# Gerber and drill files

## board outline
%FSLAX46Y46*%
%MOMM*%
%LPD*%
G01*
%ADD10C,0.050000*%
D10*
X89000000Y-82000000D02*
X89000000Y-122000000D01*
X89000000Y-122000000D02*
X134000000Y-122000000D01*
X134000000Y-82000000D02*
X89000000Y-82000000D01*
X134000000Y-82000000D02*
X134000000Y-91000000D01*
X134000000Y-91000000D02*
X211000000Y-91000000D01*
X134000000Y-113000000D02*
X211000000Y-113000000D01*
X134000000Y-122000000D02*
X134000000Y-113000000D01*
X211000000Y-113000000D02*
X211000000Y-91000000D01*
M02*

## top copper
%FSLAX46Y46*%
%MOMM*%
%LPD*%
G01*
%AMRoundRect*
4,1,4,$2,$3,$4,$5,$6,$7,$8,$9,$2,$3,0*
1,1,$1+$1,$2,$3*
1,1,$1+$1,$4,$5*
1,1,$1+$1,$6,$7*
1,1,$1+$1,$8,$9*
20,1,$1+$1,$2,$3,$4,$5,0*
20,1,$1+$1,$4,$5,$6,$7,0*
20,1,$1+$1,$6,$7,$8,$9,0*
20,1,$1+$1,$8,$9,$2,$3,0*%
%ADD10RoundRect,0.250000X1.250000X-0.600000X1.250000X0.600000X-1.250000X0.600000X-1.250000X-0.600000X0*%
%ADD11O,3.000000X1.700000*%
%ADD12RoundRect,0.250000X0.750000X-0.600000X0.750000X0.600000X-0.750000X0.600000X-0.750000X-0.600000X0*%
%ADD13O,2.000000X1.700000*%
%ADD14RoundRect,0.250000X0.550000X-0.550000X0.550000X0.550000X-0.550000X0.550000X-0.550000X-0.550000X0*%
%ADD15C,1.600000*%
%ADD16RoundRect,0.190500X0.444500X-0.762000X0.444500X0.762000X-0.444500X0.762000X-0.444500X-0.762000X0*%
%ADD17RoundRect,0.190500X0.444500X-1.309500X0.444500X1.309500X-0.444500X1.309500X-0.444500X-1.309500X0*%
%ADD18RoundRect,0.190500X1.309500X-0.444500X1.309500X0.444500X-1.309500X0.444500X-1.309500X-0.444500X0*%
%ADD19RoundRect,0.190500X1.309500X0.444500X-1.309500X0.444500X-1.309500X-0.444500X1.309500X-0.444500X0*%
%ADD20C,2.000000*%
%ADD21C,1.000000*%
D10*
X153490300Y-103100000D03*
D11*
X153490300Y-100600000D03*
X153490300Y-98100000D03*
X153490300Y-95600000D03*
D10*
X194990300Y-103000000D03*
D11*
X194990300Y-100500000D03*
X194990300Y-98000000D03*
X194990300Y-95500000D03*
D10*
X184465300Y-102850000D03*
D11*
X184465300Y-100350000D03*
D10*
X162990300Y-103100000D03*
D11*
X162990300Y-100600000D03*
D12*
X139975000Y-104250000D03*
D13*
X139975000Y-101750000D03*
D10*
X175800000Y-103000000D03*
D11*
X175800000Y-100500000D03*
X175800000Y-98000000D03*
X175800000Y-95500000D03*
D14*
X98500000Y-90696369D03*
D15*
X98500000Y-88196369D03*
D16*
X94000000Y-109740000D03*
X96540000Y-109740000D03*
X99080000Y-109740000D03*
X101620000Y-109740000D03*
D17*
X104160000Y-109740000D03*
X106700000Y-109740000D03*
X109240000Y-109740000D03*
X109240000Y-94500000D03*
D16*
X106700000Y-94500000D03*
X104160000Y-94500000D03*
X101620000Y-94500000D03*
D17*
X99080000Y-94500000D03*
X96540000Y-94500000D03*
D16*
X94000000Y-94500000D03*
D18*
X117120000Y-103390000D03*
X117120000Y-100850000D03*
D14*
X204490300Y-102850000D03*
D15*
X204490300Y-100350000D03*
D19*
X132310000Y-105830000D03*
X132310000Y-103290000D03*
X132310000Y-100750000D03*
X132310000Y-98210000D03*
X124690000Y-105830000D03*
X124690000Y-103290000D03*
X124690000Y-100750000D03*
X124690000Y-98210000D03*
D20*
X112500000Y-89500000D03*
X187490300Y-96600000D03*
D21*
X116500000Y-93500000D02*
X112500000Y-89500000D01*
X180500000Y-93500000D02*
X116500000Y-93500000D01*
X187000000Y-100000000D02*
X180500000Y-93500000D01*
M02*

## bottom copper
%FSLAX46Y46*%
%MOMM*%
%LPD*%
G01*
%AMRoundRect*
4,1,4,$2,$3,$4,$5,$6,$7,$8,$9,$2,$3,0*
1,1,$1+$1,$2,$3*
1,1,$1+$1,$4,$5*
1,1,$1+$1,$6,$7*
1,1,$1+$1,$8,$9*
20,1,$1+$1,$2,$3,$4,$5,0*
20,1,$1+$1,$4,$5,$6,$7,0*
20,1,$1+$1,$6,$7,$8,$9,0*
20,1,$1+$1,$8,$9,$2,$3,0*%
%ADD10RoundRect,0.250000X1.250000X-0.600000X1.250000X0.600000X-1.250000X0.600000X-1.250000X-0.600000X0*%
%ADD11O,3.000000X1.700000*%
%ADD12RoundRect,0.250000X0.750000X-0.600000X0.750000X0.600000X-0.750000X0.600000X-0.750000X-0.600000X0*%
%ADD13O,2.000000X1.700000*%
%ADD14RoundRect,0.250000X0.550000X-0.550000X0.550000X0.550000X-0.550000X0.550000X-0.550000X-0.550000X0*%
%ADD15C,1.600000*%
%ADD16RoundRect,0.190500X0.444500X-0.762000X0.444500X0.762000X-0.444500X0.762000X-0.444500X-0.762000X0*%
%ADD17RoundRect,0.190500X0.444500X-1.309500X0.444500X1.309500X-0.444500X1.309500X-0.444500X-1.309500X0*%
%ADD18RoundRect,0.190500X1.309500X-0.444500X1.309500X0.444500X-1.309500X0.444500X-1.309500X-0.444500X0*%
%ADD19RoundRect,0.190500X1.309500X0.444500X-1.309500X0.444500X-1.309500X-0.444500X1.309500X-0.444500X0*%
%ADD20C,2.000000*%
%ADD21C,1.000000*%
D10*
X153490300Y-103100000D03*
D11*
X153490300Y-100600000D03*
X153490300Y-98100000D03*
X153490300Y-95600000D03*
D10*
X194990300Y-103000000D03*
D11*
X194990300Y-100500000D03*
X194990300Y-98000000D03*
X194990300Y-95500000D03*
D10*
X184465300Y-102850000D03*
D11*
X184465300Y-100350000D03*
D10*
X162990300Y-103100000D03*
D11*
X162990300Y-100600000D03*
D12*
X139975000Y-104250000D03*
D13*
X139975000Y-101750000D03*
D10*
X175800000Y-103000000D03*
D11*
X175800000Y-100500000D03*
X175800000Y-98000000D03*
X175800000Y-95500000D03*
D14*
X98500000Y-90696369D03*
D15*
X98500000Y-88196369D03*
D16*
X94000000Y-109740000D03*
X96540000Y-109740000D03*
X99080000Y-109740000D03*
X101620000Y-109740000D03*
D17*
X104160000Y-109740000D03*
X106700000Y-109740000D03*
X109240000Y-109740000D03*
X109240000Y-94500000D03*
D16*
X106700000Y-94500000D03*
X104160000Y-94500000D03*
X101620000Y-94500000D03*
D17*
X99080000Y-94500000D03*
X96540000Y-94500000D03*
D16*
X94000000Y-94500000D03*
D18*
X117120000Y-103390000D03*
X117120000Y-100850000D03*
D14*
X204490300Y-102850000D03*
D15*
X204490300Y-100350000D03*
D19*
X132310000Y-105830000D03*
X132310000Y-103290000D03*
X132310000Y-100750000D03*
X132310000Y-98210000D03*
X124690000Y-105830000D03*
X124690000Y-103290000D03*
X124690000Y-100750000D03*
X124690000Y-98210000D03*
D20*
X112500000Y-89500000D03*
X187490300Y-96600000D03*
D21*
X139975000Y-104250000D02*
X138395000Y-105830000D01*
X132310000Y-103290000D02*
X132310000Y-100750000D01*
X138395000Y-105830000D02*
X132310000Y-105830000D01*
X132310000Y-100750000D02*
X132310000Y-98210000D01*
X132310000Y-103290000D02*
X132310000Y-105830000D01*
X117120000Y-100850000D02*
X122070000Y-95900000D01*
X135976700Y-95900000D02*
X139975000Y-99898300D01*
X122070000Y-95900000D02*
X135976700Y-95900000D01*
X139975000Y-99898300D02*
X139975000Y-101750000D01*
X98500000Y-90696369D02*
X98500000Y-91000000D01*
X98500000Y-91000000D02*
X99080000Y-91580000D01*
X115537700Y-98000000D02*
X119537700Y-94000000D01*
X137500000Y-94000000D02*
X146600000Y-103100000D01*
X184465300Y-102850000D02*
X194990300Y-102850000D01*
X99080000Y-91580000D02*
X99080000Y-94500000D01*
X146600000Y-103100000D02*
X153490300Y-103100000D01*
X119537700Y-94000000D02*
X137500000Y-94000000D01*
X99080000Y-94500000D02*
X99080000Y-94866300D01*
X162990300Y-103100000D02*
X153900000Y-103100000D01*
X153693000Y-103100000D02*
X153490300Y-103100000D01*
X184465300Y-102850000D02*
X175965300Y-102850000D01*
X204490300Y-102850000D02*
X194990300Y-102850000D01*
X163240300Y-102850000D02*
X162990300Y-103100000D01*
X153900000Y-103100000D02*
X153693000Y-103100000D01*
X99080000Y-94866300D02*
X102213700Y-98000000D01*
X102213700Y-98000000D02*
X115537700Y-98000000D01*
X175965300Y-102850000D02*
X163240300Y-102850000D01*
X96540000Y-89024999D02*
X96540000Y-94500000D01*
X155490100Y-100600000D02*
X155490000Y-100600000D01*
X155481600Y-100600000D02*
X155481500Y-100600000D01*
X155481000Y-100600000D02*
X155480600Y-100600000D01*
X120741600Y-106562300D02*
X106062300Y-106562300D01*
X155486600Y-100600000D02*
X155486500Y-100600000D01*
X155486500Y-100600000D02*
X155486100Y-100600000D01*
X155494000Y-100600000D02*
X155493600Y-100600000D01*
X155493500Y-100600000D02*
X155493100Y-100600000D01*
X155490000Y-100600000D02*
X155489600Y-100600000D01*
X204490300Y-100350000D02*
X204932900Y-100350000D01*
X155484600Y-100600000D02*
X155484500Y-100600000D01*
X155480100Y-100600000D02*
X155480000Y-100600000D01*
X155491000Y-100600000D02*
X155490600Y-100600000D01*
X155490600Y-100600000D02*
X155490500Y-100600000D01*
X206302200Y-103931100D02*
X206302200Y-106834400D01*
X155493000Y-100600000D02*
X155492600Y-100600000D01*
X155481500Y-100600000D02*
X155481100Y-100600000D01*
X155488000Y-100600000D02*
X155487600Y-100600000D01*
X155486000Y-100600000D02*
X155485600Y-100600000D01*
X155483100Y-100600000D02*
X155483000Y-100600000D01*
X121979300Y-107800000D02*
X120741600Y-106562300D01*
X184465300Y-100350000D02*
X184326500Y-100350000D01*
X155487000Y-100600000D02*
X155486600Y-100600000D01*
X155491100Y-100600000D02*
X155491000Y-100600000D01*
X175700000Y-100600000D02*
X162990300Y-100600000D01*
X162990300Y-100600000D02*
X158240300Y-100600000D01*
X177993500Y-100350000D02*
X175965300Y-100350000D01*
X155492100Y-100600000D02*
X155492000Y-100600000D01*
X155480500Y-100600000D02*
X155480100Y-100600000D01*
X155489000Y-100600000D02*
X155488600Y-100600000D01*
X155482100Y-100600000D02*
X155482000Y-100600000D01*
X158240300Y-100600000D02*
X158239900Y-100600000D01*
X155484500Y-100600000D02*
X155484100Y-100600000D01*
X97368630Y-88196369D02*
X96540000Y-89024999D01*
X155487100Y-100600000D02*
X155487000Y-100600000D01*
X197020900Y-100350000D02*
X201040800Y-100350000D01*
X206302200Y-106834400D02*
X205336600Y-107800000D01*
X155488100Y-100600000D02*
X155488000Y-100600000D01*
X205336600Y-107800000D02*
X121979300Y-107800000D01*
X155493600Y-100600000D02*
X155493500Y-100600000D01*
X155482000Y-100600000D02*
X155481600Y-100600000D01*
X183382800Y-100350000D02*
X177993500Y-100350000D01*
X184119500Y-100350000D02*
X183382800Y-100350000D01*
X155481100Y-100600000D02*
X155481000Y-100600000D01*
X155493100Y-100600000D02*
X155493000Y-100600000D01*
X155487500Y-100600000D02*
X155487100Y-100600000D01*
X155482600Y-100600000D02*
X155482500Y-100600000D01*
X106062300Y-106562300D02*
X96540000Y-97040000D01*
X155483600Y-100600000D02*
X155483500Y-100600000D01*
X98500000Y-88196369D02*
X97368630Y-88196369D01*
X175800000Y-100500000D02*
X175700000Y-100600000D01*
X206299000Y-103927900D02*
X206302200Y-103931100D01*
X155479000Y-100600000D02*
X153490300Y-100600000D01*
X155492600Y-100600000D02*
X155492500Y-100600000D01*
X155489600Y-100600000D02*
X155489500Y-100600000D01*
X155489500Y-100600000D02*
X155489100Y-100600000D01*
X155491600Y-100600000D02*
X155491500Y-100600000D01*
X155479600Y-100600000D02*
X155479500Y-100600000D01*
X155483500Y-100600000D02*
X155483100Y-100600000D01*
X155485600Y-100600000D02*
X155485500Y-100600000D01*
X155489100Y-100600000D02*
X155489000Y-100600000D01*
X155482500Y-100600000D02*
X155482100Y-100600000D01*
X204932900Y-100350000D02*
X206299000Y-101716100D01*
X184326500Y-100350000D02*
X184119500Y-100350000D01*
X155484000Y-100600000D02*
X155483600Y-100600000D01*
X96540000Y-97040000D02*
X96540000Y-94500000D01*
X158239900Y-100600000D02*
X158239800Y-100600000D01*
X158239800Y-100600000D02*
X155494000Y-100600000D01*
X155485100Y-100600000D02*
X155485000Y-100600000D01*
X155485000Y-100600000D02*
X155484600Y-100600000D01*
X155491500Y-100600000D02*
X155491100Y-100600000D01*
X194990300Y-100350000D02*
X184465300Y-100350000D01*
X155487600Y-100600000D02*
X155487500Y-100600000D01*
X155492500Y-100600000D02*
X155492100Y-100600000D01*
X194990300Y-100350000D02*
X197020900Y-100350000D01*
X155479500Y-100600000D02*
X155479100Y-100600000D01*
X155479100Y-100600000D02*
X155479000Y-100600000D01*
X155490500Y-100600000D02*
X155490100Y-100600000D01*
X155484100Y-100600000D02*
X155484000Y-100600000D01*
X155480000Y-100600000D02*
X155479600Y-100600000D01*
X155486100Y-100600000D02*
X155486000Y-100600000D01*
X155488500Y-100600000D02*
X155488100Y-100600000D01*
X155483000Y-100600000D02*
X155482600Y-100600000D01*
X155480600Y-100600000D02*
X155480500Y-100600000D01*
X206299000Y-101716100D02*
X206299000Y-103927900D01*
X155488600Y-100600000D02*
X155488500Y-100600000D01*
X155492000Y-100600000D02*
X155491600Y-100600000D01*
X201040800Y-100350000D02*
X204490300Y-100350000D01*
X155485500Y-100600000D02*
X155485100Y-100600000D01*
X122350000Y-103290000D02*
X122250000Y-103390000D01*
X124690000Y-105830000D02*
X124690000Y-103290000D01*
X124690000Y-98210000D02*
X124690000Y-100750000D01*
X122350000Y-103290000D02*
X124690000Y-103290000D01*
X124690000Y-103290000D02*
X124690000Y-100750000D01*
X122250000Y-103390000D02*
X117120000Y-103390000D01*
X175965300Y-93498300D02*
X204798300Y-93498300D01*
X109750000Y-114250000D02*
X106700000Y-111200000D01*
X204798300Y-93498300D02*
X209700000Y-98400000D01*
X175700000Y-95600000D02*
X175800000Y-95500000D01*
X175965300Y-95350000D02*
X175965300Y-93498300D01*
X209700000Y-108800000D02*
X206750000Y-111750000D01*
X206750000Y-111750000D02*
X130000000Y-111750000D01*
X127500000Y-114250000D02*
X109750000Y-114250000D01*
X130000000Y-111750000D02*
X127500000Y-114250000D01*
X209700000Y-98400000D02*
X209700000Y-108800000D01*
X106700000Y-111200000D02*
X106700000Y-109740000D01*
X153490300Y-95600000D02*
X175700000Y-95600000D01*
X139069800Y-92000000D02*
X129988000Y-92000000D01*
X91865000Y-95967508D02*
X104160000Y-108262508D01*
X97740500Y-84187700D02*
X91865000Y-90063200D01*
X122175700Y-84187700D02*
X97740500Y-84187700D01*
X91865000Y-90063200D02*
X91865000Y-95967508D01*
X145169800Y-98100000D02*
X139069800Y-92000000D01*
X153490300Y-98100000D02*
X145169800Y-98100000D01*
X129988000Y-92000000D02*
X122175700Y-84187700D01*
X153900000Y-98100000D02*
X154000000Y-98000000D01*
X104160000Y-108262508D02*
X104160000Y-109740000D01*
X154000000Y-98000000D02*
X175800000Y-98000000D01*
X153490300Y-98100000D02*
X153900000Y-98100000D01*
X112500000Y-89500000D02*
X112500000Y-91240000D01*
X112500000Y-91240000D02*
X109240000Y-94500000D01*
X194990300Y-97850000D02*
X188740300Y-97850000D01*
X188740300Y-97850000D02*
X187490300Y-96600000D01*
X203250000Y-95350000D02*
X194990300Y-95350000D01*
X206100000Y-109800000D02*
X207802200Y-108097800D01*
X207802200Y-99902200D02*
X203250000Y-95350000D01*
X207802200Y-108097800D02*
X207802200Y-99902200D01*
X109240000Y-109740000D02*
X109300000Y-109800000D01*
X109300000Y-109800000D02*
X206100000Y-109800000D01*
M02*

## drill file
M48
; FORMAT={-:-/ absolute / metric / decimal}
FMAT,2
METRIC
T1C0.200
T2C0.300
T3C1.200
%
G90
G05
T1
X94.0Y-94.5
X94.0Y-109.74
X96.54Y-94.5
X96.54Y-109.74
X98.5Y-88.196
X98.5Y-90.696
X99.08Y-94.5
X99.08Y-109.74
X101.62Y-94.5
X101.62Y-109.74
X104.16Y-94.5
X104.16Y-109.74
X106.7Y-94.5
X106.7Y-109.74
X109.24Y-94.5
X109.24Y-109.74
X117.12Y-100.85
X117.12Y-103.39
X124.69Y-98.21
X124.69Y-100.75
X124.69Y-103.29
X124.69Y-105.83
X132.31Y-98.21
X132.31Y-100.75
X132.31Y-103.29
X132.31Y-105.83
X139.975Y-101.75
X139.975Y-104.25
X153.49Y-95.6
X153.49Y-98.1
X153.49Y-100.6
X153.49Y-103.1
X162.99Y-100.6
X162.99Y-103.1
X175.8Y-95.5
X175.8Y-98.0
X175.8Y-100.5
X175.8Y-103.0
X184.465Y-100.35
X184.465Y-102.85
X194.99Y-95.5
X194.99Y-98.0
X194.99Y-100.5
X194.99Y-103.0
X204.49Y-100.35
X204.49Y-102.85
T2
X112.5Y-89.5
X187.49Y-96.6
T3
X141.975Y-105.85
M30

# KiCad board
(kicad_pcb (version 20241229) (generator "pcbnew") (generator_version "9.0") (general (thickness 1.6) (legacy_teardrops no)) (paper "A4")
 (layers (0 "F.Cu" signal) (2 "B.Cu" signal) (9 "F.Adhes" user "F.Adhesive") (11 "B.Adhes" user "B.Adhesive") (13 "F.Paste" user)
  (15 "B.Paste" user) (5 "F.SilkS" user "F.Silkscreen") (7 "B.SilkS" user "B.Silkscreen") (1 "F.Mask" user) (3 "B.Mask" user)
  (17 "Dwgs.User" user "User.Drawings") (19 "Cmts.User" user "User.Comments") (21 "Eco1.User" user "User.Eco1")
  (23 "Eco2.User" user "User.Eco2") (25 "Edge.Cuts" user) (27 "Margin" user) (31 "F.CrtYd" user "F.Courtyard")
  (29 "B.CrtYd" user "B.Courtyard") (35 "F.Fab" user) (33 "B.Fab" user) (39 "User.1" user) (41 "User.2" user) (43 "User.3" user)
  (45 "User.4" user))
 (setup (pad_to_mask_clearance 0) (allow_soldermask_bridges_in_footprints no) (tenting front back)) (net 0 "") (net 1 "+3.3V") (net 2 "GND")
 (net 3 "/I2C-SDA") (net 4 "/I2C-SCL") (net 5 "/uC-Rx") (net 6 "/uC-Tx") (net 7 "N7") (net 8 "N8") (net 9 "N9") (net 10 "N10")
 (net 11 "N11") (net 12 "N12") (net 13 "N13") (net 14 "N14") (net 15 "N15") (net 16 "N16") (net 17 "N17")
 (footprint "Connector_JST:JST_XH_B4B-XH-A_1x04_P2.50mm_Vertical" (layer "F.Cu") (at 153.4903 103.1 90)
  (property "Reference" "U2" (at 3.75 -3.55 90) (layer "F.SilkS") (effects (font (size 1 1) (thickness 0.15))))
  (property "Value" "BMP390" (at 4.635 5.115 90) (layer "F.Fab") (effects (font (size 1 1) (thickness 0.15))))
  (pad "1" thru_hole roundrect (at 0 0 90) (size 1.7 3) (drill 0.2) (layers "*.Cu" "*.Mask") (remove_unused_layers no)
   (roundrect_rratio 0.147059) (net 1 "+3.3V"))
  (pad "2" thru_hole oval (at 2.5 0 90) (size 1.7 3) (drill 0.2) (layers "*.Cu" "*.Mask") (remove_unused_layers no) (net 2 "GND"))
  (pad "3" thru_hole oval (at 5 0 90) (size 1.7 3) (drill 0.2) (layers "*.Cu" "*.Mask") (remove_unused_layers no) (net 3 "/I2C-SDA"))
  (pad "4" thru_hole oval (at 7.5 0 90) (size 1.7 3) (drill 0.2) (layers "*.Cu" "*.Mask") (remove_unused_layers no) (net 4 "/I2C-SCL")))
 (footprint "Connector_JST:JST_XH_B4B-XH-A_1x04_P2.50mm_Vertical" (layer "F.Cu") (at 194.9903 103 90)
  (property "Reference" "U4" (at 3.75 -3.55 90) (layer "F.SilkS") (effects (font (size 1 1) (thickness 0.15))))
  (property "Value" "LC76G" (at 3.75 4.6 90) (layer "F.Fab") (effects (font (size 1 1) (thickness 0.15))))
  (pad "1" thru_hole roundrect (at 0 0 90) (size 1.7 3) (drill 0.2) (layers "*.Cu" "*.Mask") (remove_unused_layers no)
   (roundrect_rratio 0.147059) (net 1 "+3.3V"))
  (pad "2" thru_hole oval (at 2.5 0 90) (size 1.7 3) (drill 0.2) (layers "*.Cu" "*.Mask") (remove_unused_layers no) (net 2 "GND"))
  (pad "3" thru_hole oval (at 5 0 90) (size 1.7 3) (drill 0.2) (layers "*.Cu" "*.Mask") (remove_unused_layers no) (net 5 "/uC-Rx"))
  (pad "4" thru_hole oval (at 7.5 0 90) (size 1.7 3) (drill 0.2) (layers "*.Cu" "*.Mask") (remove_unused_layers no) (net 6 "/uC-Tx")))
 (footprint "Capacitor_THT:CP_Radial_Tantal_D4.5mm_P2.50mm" (layer "F.Cu") (at 184.4653 102.85 90)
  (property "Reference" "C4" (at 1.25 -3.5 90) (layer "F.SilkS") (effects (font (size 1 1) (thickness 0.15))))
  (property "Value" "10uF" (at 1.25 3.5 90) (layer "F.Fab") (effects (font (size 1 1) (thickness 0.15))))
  (pad "1" thru_hole roundrect (at 0 0 90) (size 1.7 3) (drill 0.2) (layers "*.Cu" "*.Mask") (remove_unused_layers no)
   (roundrect_rratio 0.147059) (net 1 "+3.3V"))
  (pad "2" thru_hole oval (at 2.5 0 90) (size 1.7 3) (drill 0.2) (layers "*.Cu" "*.Mask") (remove_unused_layers no) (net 2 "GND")))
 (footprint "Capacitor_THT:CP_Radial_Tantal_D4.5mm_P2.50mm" (layer "F.Cu") (at 162.9903 103.1 90)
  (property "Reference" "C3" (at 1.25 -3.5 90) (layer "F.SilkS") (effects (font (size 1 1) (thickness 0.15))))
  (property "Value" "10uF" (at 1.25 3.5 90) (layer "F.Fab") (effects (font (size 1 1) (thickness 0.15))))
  (pad "1" thru_hole roundrect (at 0 0 90) (size 1.7 3) (drill 0.2) (layers "*.Cu" "*.Mask") (remove_unused_layers no)
   (roundrect_rratio 0.147059) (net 1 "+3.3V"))
  (pad "2" thru_hole oval (at 2.5 0 90) (size 1.7 3) (drill 0.2) (layers "*.Cu" "*.Mask") (remove_unused_layers no) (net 2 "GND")))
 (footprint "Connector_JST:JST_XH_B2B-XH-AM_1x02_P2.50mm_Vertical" (layer "F.Cu") (at 139.975 104.25 90)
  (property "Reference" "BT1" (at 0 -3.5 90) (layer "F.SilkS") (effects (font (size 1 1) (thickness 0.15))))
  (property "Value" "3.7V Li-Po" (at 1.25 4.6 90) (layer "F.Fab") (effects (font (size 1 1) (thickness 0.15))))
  (pad "" np_thru_hole circle (at -1.6 2 90) (size 1.2 1.2) (drill 1.2) (layers "*.Cu" "*.Mask"))
  (pad "1" thru_hole roundrect (at 0 0 90) (size 1.7 2) (drill 0.2) (layers "*.Cu" "*.Mask") (remove_unused_layers no)
   (roundrect_rratio 0.147059) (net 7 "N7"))
  (pad "2" thru_hole oval (at 2.5 0 90) (size 1.7 2) (drill 0.2) (layers "*.Cu" "*.Mask") (remove_unused_layers no) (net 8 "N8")))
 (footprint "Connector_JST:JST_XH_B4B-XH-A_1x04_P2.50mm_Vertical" (layer "F.Cu") (at 175.8 103 90)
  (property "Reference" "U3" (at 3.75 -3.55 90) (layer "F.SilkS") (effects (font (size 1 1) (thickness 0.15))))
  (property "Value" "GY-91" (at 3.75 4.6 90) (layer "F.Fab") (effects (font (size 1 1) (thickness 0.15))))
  (pad "1" thru_hole roundrect (at 0 0 90) (size 1.7 3) (drill 0.2) (layers "*.Cu" "*.Mask") (remove_unused_layers no)
   (roundrect_rratio 0.147059) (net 1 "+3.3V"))
  (pad "2" thru_hole oval (at 2.5 0 90) (size 1.7 3) (drill 0.2) (layers "*.Cu" "*.Mask") (remove_unused_layers no) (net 2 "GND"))
  (pad "3" thru_hole oval (at 5 0 90) (size 1.7 3) (drill 0.2) (layers "*.Cu" "*.Mask") (remove_unused_layers no) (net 3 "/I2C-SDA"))
  (pad "4" thru_hole oval (at 7.5 0 90) (size 1.7 3) (drill 0.2) (layers "*.Cu" "*.Mask") (remove_unused_layers no) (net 4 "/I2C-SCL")))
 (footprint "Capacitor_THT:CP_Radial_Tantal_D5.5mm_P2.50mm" (layer "F.Cu") (at 98.5 90.696369 90)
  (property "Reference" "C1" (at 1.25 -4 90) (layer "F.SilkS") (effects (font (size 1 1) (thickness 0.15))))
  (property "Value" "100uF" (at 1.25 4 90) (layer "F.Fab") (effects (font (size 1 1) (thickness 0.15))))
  (pad "1" thru_hole roundrect (at 0 0 90) (size 1.6 1.6) (drill 0.2) (layers "*.Cu" "*.Mask") (remove_unused_layers no)
   (roundrect_rratio 0.15625) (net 1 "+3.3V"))
  (pad "2" thru_hole circle (at 2.5 0 90) (size 1.6 1.6) (drill 0.2) (layers "*.Cu" "*.Mask") (remove_unused_layers no) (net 2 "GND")))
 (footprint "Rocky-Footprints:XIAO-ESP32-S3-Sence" (layer "F.Cu") (at 101.62 102.12 90)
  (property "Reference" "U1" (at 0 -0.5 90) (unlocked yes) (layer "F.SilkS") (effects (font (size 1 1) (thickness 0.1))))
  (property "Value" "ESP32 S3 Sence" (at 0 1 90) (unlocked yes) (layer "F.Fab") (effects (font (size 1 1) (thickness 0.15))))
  (pad "1" thru_hole roundrect (at -7.62 -7.62 90) (size 1.905 1.27) (drill 0.2) (layers "*.Cu" "*.Mask") (remove_unused_layers no)
   (roundrect_rratio 0.15) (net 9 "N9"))
  (pad "2" thru_hole roundrect (at -7.62 -5.08 90) (size 1.905 1.27) (drill 0.2) (layers "*.Cu" "*.Mask") (remove_unused_layers no)
   (roundrect_rratio 0.15) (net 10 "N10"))
  (pad "3" thru_hole roundrect (at -7.62 -2.54 90) (size 1.905 1.27) (drill 0.2) (layers "*.Cu" "*.Mask") (remove_unused_layers no)
   (roundrect_rratio 0.15) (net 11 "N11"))
  (pad "4" thru_hole roundrect (at -7.62 0 90) (size 1.905 1.27) (drill 0.2) (layers "*.Cu" "*.Mask") (remove_unused_layers no)
   (roundrect_rratio 0.15) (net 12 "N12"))
  (pad "5" thru_hole roundrect (at -7.62 2.54 90) (size 3 1.27) (drill 0.2) (layers "*.Cu" "*.Mask") (remove_unused_layers no)
   (roundrect_rratio 0.15) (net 3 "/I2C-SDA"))
  (pad "6" thru_hole roundrect (at -7.62 5.08 90) (size 3 1.27) (drill 0.2) (layers "*.Cu" "*.Mask") (remove_unused_layers no)
   (roundrect_rratio 0.15) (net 4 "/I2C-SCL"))
  (pad "7" thru_hole roundrect (at -7.62 7.62 90) (size 3 1.27) (drill 0.2) (layers "*.Cu" "*.Mask") (remove_unused_layers no)
   (roundrect_rratio 0.15) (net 6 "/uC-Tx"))
  (pad "8" thru_hole roundrect (at 7.62 7.62 90) (size 3 1.27) (drill 0.2) (layers "*.Cu" "*.Mask") (remove_unused_layers no)
   (roundrect_rratio 0.15) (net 5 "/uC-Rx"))
  (pad "9" thru_hole roundrect (at 7.62 5.08 90) (size 1.905 1.27) (drill 0.2) (layers "*.Cu" "*.Mask") (remove_unused_layers no)
   (roundrect_rratio 0.15) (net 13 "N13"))
  (pad "10" thru_hole roundrect (at 7.62 2.54 90) (size 1.905 1.27) (drill 0.2) (layers "*.Cu" "*.Mask") (remove_unused_layers no)
   (roundrect_rratio 0.15) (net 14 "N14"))
  (pad "11" thru_hole roundrect (at 7.62 0 90) (size 1.905 1.27) (drill 0.2) (layers "*.Cu" "*.Mask") (remove_unused_layers no)
   (roundrect_rratio 0.15) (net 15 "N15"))
  (pad "12" thru_hole roundrect (at 7.62 -2.54 90) (size 3 1.27) (drill 0.2) (layers "*.Cu" "*.Mask") (remove_unused_layers no)
   (roundrect_rratio 0.15) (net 1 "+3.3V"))
  (pad "13" thru_hole roundrect (at 7.62 -5.08 90) (size 3 1.27) (drill 0.2) (layers "*.Cu" "*.Mask") (remove_unused_layers no)
   (roundrect_rratio 0.15) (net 2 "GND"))
  (pad "14" thru_hole roundrect (at 7.62 -7.62 90) (size 1.905 1.27) (drill 0.2) (layers "*.Cu" "*.Mask") (remove_unused_layers no)
   (roundrect_rratio 0.15) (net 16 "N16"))
  (pad "15" thru_hole roundrect (at -1.27 15.5 90) (size 1.27 3) (drill 0.2) (layers "*.Cu" "*.Mask") (remove_unused_layers no)
   (roundrect_rratio 0.15) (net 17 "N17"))
  (pad "16" thru_hole roundrect (at 1.27 15.5 90) (size 1.27 3) (drill 0.2) (layers "*.Cu" "*.Mask") (remove_unused_layers no)
   (roundrect_rratio 0.15) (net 8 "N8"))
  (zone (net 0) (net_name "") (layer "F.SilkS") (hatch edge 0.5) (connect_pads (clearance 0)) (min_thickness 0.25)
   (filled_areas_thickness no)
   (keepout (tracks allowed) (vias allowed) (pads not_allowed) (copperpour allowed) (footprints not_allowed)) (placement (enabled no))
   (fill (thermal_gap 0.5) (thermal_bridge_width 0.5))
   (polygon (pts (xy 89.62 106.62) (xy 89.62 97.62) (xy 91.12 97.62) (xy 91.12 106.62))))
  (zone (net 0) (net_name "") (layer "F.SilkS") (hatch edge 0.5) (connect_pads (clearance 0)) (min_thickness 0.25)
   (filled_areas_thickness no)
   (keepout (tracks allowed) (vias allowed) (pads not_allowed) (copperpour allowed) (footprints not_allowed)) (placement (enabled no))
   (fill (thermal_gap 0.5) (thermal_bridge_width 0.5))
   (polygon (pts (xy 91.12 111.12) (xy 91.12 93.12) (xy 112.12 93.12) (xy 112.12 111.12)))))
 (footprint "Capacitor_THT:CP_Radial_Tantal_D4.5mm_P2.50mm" (layer "F.Cu") (at 204.4903 102.85 90)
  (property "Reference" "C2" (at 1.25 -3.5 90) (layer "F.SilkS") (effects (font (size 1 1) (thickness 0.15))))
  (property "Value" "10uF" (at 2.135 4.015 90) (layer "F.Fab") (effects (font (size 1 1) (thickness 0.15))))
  (pad "1" thru_hole roundrect (at 0 0 90) (size 1.6 1.6) (drill 0.2) (layers "*.Cu" "*.Mask") (remove_unused_layers no)
   (roundrect_rratio 0.15625) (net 1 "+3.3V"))
  (pad "2" thru_hole circle (at 2.5 0 90) (size 1.6 1.6) (drill 0.2) (layers "*.Cu" "*.Mask") (remove_unused_layers no) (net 2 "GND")))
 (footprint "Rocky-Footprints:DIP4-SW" (layer "F.Cu") (at 128.5 100.75 180)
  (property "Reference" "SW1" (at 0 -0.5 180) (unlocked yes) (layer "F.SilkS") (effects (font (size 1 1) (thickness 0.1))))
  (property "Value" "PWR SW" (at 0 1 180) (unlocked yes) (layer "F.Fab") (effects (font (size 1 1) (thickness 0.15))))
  (pad "1" thru_hole roundrect (at -3.81 -5.08 180) (size 3 1.27) (drill 0.2) (layers "*.Cu" "*.Mask") (remove_unused_layers no)
   (roundrect_rratio 0.15) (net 7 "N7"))
  (pad "1" thru_hole roundrect (at -3.81 -2.54 180) (size 3 1.27) (drill 0.2) (layers "*.Cu" "*.Mask") (remove_unused_layers no)
   (roundrect_rratio 0.15) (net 7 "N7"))
  (pad "1" thru_hole roundrect (at -3.81 0 180) (size 3 1.27) (drill 0.2) (layers "*.Cu" "*.Mask") (remove_unused_layers no)
   (roundrect_rratio 0.15) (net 7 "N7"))
  (pad "1" thru_hole roundrect (at -3.81 2.54 180) (size 3 1.27) (drill 0.2) (layers "*.Cu" "*.Mask") (remove_unused_layers no)
   (roundrect_rratio 0.15) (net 7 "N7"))
  (pad "2" thru_hole roundrect (at 3.81 -5.08 180) (size 3 1.27) (drill 0.2) (layers "*.Cu" "*.Mask") (remove_unused_layers no)
   (roundrect_rratio 0.15) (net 17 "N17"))
  (pad "2" thru_hole roundrect (at 3.81 -2.54 180) (size 3 1.27) (drill 0.2) (layers "*.Cu" "*.Mask") (remove_unused_layers no)
   (roundrect_rratio 0.15) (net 17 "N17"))
  (pad "2" thru_hole roundrect (at 3.81 0 180) (size 3 1.27) (drill 0.2) (layers "*.Cu" "*.Mask") (remove_unused_layers no)
   (roundrect_rratio 0.15) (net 17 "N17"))
  (pad "2" thru_hole roundrect (at 3.81 2.54 180) (size 3 1.27) (drill 0.2) (layers "*.Cu" "*.Mask") (remove_unused_layers no)
   (roundrect_rratio 0.15) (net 17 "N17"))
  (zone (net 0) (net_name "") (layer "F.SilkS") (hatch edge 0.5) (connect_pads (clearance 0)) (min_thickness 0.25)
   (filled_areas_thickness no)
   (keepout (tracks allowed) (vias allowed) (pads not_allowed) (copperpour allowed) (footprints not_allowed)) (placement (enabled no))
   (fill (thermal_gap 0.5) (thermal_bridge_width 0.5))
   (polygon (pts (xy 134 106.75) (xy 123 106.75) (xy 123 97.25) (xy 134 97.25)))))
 (gr_line (start 89 82) (end 89 122) (stroke (width 0.05) (type default)) (layer "Edge.Cuts"))
 (gr_line (start 89 122) (end 134 122) (stroke (width 0.05) (type default)) (layer "Edge.Cuts"))
 (gr_line (start 134 82) (end 89 82) (stroke (width 0.05) (type default)) (layer "Edge.Cuts"))
 (gr_line (start 134 82) (end 134 91) (stroke (width 0.05) (type default)) (layer "Edge.Cuts"))
 (gr_line (start 134 91) (end 211 91) (stroke (width 0.05) (type default)) (layer "Edge.Cuts"))
 (gr_line (start 134 113) (end 211 113) (stroke (width 0.05) (type default)) (layer "Edge.Cuts"))
 (gr_line (start 134 122) (end 134 113) (stroke (width 0.05) (type default)) (layer "Edge.Cuts"))
 (gr_line (start 211 113) (end 211 91) (stroke (width 0.05) (type default)) (layer "Edge.Cuts"))
 (segment (start 139.975 104.25) (end 138.395 105.83) (width 1) (layer "B.Cu") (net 7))
 (segment (start 132.31 103.29) (end 132.31 100.75) (width 1) (layer "B.Cu") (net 7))
 (segment (start 138.395 105.83) (end 132.31 105.83) (width 1) (layer "B.Cu") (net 7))
 (segment (start 132.31 100.75) (end 132.31 98.21) (width 1) (layer "B.Cu") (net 7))
 (segment (start 132.31 103.29) (end 132.31 105.83) (width 1) (layer "B.Cu") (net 7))
 (segment (start 117.12 100.85) (end 122.07 95.9) (width 1) (layer "B.Cu") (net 8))
 (segment (start 135.9767 95.9) (end 139.975 99.8983) (width 1) (layer "B.Cu") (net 8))
 (segment (start 122.07 95.9) (end 135.9767 95.9) (width 1) (layer "B.Cu") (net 8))
 (segment (start 139.975 99.8983) (end 139.975 101.75) (width 1) (layer "B.Cu") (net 8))
 (segment (start 98.5 90.696369) (end 98.5 91) (width 1) (layer "B.Cu") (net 1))
 (segment (start 98.5 91) (end 99.08 91.58) (width 1) (layer "B.Cu") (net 1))
 (segment (start 115.5377 98) (end 119.5377 94) (width 1) (layer "B.Cu") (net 1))
 (segment (start 137.5 94) (end 146.6 103.1) (width 1) (layer "B.Cu") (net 1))
 (segment (start 184.4653 102.85) (end 194.9903 102.85) (width 1) (layer "B.Cu") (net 1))
 (segment (start 99.08 91.58) (end 99.08 94.5) (width 1) (layer "B.Cu") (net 1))
 (segment (start 146.6 103.1) (end 153.4903 103.1) (width 1) (layer "B.Cu") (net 1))
 (segment (start 119.5377 94) (end 137.5 94) (width 1) (layer "B.Cu") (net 1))
 (segment (start 99.08 94.5) (end 99.08 94.8663) (width 1) (layer "B.Cu") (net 1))
 (segment (start 162.9903 103.1) (end 153.9 103.1) (width 1) (layer "B.Cu") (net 1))
 (segment (start 153.693 103.1) (end 153.4903 103.1) (width 1) (layer "B.Cu") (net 1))
 (segment (start 184.4653 102.85) (end 175.9653 102.85) (width 1) (layer "B.Cu") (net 1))
 (segment (start 204.4903 102.85) (end 194.9903 102.85) (width 1) (layer "B.Cu") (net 1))
 (segment (start 163.2403 102.85) (end 162.9903 103.1) (width 1) (layer "B.Cu") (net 1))
 (segment (start 153.9 103.1) (end 153.693 103.1) (width 1) (layer "B.Cu") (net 1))
 (segment (start 99.08 94.8663) (end 102.2137 98) (width 1) (layer "B.Cu") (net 1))
 (segment (start 102.2137 98) (end 115.5377 98) (width 1) (layer "B.Cu") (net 1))
 (segment (start 175.9653 102.85) (end 163.2403 102.85) (width 1) (layer "B.Cu") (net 1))
 (segment (start 96.54 89.024999) (end 96.54 94.5) (width 1) (layer "B.Cu") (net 2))
 (segment (start 155.4901 100.6) (end 155.49 100.6) (width 1) (layer "B.Cu") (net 2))
 (segment (start 155.4816 100.6) (end 155.4815 100.6) (width 1) (layer "B.Cu") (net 2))
 (segment (start 155.481 100.6) (end 155.4806 100.6) (width 1) (layer "B.Cu") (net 2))
 (segment (start 120.7416 106.5623) (end 106.0623 106.5623) (width 1) (layer "B.Cu") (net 2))
 (segment (start 155.4866 100.6) (end 155.4865 100.6) (width 1) (layer "B.Cu") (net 2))
 (segment (start 155.4865 100.6) (end 155.4861 100.6) (width 1) (layer "B.Cu") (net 2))
 (segment (start 155.494 100.6) (end 155.4936 100.6) (width 1) (layer "B.Cu") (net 2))
 (segment (start 155.4935 100.6) (end 155.4931 100.6) (width 1) (layer "B.Cu") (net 2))
 (segment (start 155.49 100.6) (end 155.4896 100.6) (width 1) (layer "B.Cu") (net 2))
 (segment (start 204.4903 100.35) (end 204.9329 100.35) (width 1) (layer "B.Cu") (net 2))
 (segment (start 155.4846 100.6) (end 155.4845 100.6) (width 1) (layer "B.Cu") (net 2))
 (segment (start 155.4801 100.6) (end 155.48 100.6) (width 1) (layer "B.Cu") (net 2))
 (segment (start 155.491 100.6) (end 155.4906 100.6) (width 1) (layer "B.Cu") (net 2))
 (segment (start 155.4906 100.6) (end 155.4905 100.6) (width 1) (layer "B.Cu") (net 2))
 (segment (start 206.3022 103.9311) (end 206.3022 106.8344) (width 1) (layer "B.Cu") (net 2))
 (segment (start 155.493 100.6) (end 155.4926 100.6) (width 1) (layer "B.Cu") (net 2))
 (segment (start 155.4815 100.6) (end 155.4811 100.6) (width 1) (layer "B.Cu") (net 2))
 (segment (start 155.488 100.6) (end 155.4876 100.6) (width 1) (layer "B.Cu") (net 2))
 (segment (start 155.486 100.6) (end 155.4856 100.6) (width 1) (layer "B.Cu") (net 2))
 (segment (start 155.4831 100.6) (end 155.483 100.6) (width 1) (layer "B.Cu") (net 2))
 (segment (start 121.9793 107.8) (end 120.7416 106.5623) (width 1) (layer "B.Cu") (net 2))
 (segment (start 184.4653 100.35) (end 184.3265 100.35) (width 1) (layer "B.Cu") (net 2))
 (segment (start 155.487 100.6) (end 155.4866 100.6) (width 1) (layer "B.Cu") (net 2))
 (segment (start 155.4911 100.6) (end 155.491 100.6) (width 1) (layer "B.Cu") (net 2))
 (segment (start 175.7 100.6) (end 162.9903 100.6) (width 1) (layer "B.Cu") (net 2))
 (segment (start 162.9903 100.6) (end 158.2403 100.6) (width 1) (layer "B.Cu") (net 2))
 (segment (start 177.9935 100.35) (end 175.9653 100.35) (width 1) (layer "B.Cu") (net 2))
 (segment (start 155.4921 100.6) (end 155.492 100.6) (width 1) (layer "B.Cu") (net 2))
 (segment (start 155.4805 100.6) (end 155.4801 100.6) (width 1) (layer "B.Cu") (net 2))
 (segment (start 155.489 100.6) (end 155.4886 100.6) (width 1) (layer "B.Cu") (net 2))
 (segment (start 155.4821 100.6) (end 155.482 100.6) (width 1) (layer "B.Cu") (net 2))
 (segment (start 158.2403 100.6) (end 158.2399 100.6) (width 1) (layer "B.Cu") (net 2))
 (segment (start 155.4845 100.6) (end 155.4841 100.6) (width 1) (layer "B.Cu") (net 2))
 (segment (start 97.36863 88.196369) (end 96.54 89.024999) (width 1) (layer "B.Cu") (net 2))
 (segment (start 155.4871 100.6) (end 155.487 100.6) (width 1) (layer "B.Cu") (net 2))
 (segment (start 197.0209 100.35) (end 201.0408 100.35) (width 1) (layer "B.Cu") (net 2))
 (segment (start 206.3022 106.8344) (end 205.3366 107.8) (width 1) (layer "B.Cu") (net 2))
 (segment (start 155.4881 100.6) (end 155.488 100.6) (width 1) (layer "B.Cu") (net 2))
 (segment (start 205.3366 107.8) (end 121.9793 107.8) (width 1) (layer "B.Cu") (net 2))
 (segment (start 155.4936 100.6) (end 155.4935 100.6) (width 1) (layer "B.Cu") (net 2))
 (segment (start 155.482 100.6) (end 155.4816 100.6) (width 1) (layer "B.Cu") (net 2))
 (segment (start 183.3828 100.35) (end 177.9935 100.35) (width 1) (layer "B.Cu") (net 2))
 (segment (start 184.1195 100.35) (end 183.3828 100.35) (width 1) (layer "B.Cu") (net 2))
 (segment (start 155.4811 100.6) (end 155.481 100.6) (width 1) (layer "B.Cu") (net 2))
 (segment (start 155.4931 100.6) (end 155.493 100.6) (width 1) (layer "B.Cu") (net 2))
 (segment (start 155.4875 100.6) (end 155.4871 100.6) (width 1) (layer "B.Cu") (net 2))
 (segment (start 155.4826 100.6) (end 155.4825 100.6) (width 1) (layer "B.Cu") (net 2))
 (segment (start 106.0623 106.5623) (end 96.54 97.04) (width 1) (layer "B.Cu") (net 2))
 (segment (start 155.4836 100.6) (end 155.4835 100.6) (width 1) (layer "B.Cu") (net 2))
 (segment (start 98.5 88.196369) (end 97.36863 88.196369) (width 1) (layer "B.Cu") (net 2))
 (segment (start 175.8 100.5) (end 175.7 100.6) (width 1) (layer "B.Cu") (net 2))
 (segment (start 206.299 103.9279) (end 206.3022 103.9311) (width 1) (layer "B.Cu") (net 2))
 (segment (start 155.479 100.6) (end 153.4903 100.6) (width 1) (layer "B.Cu") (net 2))
 (segment (start 155.4926 100.6) (end 155.4925 100.6) (width 1) (layer "B.Cu") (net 2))
 (segment (start 155.4896 100.6) (end 155.4895 100.6) (width 1) (layer "B.Cu") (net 2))
 (segment (start 155.4895 100.6) (end 155.4891 100.6) (width 1) (layer "B.Cu") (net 2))
 (segment (start 155.4916 100.6) (end 155.4915 100.6) (width 1) (layer "B.Cu") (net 2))
 (segment (start 155.4796 100.6) (end 155.4795 100.6) (width 1) (layer "B.Cu") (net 2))
 (segment (start 155.4835 100.6) (end 155.4831 100.6) (width 1) (layer "B.Cu") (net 2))
 (segment (start 155.4856 100.6) (end 155.4855 100.6) (width 1) (layer "B.Cu") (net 2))
 (segment (start 155.4891 100.6) (end 155.489 100.6) (width 1) (layer "B.Cu") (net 2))
 (segment (start 155.4825 100.6) (end 155.4821 100.6) (width 1) (layer "B.Cu") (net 2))
 (segment (start 204.9329 100.35) (end 206.299 101.7161) (width 1) (layer "B.Cu") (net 2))
 (segment (start 184.3265 100.35) (end 184.1195 100.35) (width 1) (layer "B.Cu") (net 2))
 (segment (start 155.484 100.6) (end 155.4836 100.6) (width 1) (layer "B.Cu") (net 2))
 (segment (start 96.54 97.04) (end 96.54 94.5) (width 1) (layer "B.Cu") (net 2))
 (segment (start 158.2399 100.6) (end 158.2398 100.6) (width 1) (layer "B.Cu") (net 2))
 (segment (start 158.2398 100.6) (end 155.494 100.6) (width 1) (layer "B.Cu") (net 2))
 (segment (start 155.4851 100.6) (end 155.485 100.6) (width 1) (layer "B.Cu") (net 2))
 (segment (start 155.485 100.6) (end 155.4846 100.6) (width 1) (layer "B.Cu") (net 2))
 (segment (start 155.4915 100.6) (end 155.4911 100.6) (width 1) (layer "B.Cu") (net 2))
 (segment (start 194.9903 100.35) (end 184.4653 100.35) (width 1) (layer "B.Cu") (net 2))
 (segment (start 155.4876 100.6) (end 155.4875 100.6) (width 1) (layer "B.Cu") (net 2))
 (segment (start 155.4925 100.6) (end 155.4921 100.6) (width 1) (layer "B.Cu") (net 2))
 (segment (start 194.9903 100.35) (end 197.0209 100.35) (width 1) (layer "B.Cu") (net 2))
 (segment (start 155.4795 100.6) (end 155.4791 100.6) (width 1) (layer "B.Cu") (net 2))
 (segment (start 155.4791 100.6) (end 155.479 100.6) (width 1) (layer "B.Cu") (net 2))
 (segment (start 155.4905 100.6) (end 155.4901 100.6) (width 1) (layer "B.Cu") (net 2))
 (segment (start 155.4841 100.6) (end 155.484 100.6) (width 1) (layer "B.Cu") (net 2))
 (segment (start 155.48 100.6) (end 155.4796 100.6) (width 1) (layer "B.Cu") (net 2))
 (segment (start 155.4861 100.6) (end 155.486 100.6) (width 1) (layer "B.Cu") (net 2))
 (segment (start 155.4885 100.6) (end 155.4881 100.6) (width 1) (layer "B.Cu") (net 2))
 (segment (start 155.483 100.6) (end 155.4826 100.6) (width 1) (layer "B.Cu") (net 2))
 (segment (start 155.4806 100.6) (end 155.4805 100.6) (width 1) (layer "B.Cu") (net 2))
 (segment (start 206.299 101.7161) (end 206.299 103.9279) (width 1) (layer "B.Cu") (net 2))
 (segment (start 155.4886 100.6) (end 155.4885 100.6) (width 1) (layer "B.Cu") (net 2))
 (segment (start 155.492 100.6) (end 155.4916 100.6) (width 1) (layer "B.Cu") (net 2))
 (segment (start 201.0408 100.35) (end 204.4903 100.35) (width 1) (layer "B.Cu") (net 2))
 (segment (start 155.4855 100.6) (end 155.4851 100.6) (width 1) (layer "B.Cu") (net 2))
 (segment (start 122.35 103.29) (end 122.25 103.39) (width 1) (layer "B.Cu") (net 17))
 (segment (start 124.69 105.83) (end 124.69 103.29) (width 1) (layer "B.Cu") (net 17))
 (segment (start 124.69 98.21) (end 124.69 100.75) (width 1) (layer "B.Cu") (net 17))
 (segment (start 122.35 103.29) (end 124.69 103.29) (width 1) (layer "B.Cu") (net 17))
 (segment (start 124.69 103.29) (end 124.69 100.75) (width 1) (layer "B.Cu") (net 17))
 (segment (start 122.25 103.39) (end 117.12 103.39) (width 1) (layer "B.Cu") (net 17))
 (segment (start 175.9653 93.4983) (end 204.7983 93.4983) (width 1) (layer "B.Cu") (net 4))
 (segment (start 109.75 114.25) (end 106.7 111.2) (width 1) (layer "B.Cu") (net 4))
 (segment (start 204.7983 93.4983) (end 209.7 98.4) (width 1) (layer "B.Cu") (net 4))
 (segment (start 175.7 95.6) (end 175.8 95.5) (width 1) (layer "B.Cu") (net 4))
 (segment (start 175.9653 95.35) (end 175.9653 93.4983) (width 1) (layer "B.Cu") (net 4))
 (segment (start 209.7 108.8) (end 206.75 111.75) (width 1) (layer "B.Cu") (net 4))
 (segment (start 206.75 111.75) (end 130 111.75) (width 1) (layer "B.Cu") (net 4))
 (segment (start 127.5 114.25) (end 109.75 114.25) (width 1) (layer "B.Cu") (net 4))
 (segment (start 130 111.75) (end 127.5 114.25) (width 1) (layer "B.Cu") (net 4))
 (segment (start 209.7 98.4) (end 209.7 108.8) (width 1) (layer "B.Cu") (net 4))
 (segment (start 106.7 111.2) (end 106.7 109.74) (width 1) (layer "B.Cu") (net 4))
 (segment (start 153.4903 95.6) (end 175.7 95.6) (width 1) (layer "B.Cu") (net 4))
 (segment (start 139.0698 92) (end 129.988 92) (width 1) (layer "B.Cu") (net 3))
 (segment (start 91.865 95.967508) (end 104.16 108.262508) (width 1) (layer "B.Cu") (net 3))
 (segment (start 97.7405 84.1877) (end 91.865 90.0632) (width 1) (layer "B.Cu") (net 3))
 (segment (start 122.1757 84.1877) (end 97.7405 84.1877) (width 1) (layer "B.Cu") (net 3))
 (segment (start 91.865 90.0632) (end 91.865 95.967508) (width 1) (layer "B.Cu") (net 3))
 (segment (start 145.1698 98.1) (end 139.0698 92) (width 1) (layer "B.Cu") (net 3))
 (segment (start 153.4903 98.1) (end 145.1698 98.1) (width 1) (layer "B.Cu") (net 3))
 (segment (start 129.988 92) (end 122.1757 84.1877) (width 1) (layer "B.Cu") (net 3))
 (segment (start 153.9 98.1) (end 154 98) (width 1) (layer "B.Cu") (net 3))
 (segment (start 104.16 108.262508) (end 104.16 109.74) (width 1) (layer "B.Cu") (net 3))
 (segment (start 154 98) (end 175.8 98) (width 1) (layer "B.Cu") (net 3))
 (segment (start 153.4903 98.1) (end 153.9 98.1) (width 1) (layer "B.Cu") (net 3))
 (segment (start 116.5 93.5) (end 112.5 89.5) (width 1) (layer "F.Cu") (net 5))
 (segment (start 180.5 93.5) (end 116.5 93.5) (width 1) (layer "F.Cu") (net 5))
 (segment (start 187 100) (end 180.5 93.5) (width 1) (layer "F.Cu") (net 5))
 (via (at 112.5 89.5) (size 2) (drill 0.3) (layers "F.Cu" "B.Cu") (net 5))
 (via (at 187.4903 96.6) (size 2) (drill 0.3) (layers "F.Cu" "B.Cu") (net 5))
 (segment (start 112.5 89.5) (end 112.5 91.24) (width 1) (layer "B.Cu") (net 5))
 (segment (start 112.5 91.24) (end 109.24 94.5) (width 1) (layer "B.Cu") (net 5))
 (segment (start 194.9903 97.85) (end 188.7403 97.85) (width 1) (layer "B.Cu") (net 5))
 (segment (start 188.7403 97.85) (end 187.4903 96.6) (width 1) (layer "B.Cu") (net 5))
 (segment (start 203.25 95.35) (end 194.9903 95.35) (width 1) (layer "B.Cu") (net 6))
 (segment (start 206.1 109.8) (end 207.8022 108.0978) (width 1) (layer "B.Cu") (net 6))
 (segment (start 207.8022 99.9022) (end 203.25 95.35) (width 1) (layer "B.Cu") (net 6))
 (segment (start 207.8022 108.0978) (end 207.8022 99.9022) (width 1) (layer "B.Cu") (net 6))
 (segment (start 109.24 109.74) (end 109.3 109.8) (width 1) (layer "B.Cu") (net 6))
 (segment (start 109.3 109.8) (end 206.1 109.8) (width 1) (layer "B.Cu") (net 6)))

